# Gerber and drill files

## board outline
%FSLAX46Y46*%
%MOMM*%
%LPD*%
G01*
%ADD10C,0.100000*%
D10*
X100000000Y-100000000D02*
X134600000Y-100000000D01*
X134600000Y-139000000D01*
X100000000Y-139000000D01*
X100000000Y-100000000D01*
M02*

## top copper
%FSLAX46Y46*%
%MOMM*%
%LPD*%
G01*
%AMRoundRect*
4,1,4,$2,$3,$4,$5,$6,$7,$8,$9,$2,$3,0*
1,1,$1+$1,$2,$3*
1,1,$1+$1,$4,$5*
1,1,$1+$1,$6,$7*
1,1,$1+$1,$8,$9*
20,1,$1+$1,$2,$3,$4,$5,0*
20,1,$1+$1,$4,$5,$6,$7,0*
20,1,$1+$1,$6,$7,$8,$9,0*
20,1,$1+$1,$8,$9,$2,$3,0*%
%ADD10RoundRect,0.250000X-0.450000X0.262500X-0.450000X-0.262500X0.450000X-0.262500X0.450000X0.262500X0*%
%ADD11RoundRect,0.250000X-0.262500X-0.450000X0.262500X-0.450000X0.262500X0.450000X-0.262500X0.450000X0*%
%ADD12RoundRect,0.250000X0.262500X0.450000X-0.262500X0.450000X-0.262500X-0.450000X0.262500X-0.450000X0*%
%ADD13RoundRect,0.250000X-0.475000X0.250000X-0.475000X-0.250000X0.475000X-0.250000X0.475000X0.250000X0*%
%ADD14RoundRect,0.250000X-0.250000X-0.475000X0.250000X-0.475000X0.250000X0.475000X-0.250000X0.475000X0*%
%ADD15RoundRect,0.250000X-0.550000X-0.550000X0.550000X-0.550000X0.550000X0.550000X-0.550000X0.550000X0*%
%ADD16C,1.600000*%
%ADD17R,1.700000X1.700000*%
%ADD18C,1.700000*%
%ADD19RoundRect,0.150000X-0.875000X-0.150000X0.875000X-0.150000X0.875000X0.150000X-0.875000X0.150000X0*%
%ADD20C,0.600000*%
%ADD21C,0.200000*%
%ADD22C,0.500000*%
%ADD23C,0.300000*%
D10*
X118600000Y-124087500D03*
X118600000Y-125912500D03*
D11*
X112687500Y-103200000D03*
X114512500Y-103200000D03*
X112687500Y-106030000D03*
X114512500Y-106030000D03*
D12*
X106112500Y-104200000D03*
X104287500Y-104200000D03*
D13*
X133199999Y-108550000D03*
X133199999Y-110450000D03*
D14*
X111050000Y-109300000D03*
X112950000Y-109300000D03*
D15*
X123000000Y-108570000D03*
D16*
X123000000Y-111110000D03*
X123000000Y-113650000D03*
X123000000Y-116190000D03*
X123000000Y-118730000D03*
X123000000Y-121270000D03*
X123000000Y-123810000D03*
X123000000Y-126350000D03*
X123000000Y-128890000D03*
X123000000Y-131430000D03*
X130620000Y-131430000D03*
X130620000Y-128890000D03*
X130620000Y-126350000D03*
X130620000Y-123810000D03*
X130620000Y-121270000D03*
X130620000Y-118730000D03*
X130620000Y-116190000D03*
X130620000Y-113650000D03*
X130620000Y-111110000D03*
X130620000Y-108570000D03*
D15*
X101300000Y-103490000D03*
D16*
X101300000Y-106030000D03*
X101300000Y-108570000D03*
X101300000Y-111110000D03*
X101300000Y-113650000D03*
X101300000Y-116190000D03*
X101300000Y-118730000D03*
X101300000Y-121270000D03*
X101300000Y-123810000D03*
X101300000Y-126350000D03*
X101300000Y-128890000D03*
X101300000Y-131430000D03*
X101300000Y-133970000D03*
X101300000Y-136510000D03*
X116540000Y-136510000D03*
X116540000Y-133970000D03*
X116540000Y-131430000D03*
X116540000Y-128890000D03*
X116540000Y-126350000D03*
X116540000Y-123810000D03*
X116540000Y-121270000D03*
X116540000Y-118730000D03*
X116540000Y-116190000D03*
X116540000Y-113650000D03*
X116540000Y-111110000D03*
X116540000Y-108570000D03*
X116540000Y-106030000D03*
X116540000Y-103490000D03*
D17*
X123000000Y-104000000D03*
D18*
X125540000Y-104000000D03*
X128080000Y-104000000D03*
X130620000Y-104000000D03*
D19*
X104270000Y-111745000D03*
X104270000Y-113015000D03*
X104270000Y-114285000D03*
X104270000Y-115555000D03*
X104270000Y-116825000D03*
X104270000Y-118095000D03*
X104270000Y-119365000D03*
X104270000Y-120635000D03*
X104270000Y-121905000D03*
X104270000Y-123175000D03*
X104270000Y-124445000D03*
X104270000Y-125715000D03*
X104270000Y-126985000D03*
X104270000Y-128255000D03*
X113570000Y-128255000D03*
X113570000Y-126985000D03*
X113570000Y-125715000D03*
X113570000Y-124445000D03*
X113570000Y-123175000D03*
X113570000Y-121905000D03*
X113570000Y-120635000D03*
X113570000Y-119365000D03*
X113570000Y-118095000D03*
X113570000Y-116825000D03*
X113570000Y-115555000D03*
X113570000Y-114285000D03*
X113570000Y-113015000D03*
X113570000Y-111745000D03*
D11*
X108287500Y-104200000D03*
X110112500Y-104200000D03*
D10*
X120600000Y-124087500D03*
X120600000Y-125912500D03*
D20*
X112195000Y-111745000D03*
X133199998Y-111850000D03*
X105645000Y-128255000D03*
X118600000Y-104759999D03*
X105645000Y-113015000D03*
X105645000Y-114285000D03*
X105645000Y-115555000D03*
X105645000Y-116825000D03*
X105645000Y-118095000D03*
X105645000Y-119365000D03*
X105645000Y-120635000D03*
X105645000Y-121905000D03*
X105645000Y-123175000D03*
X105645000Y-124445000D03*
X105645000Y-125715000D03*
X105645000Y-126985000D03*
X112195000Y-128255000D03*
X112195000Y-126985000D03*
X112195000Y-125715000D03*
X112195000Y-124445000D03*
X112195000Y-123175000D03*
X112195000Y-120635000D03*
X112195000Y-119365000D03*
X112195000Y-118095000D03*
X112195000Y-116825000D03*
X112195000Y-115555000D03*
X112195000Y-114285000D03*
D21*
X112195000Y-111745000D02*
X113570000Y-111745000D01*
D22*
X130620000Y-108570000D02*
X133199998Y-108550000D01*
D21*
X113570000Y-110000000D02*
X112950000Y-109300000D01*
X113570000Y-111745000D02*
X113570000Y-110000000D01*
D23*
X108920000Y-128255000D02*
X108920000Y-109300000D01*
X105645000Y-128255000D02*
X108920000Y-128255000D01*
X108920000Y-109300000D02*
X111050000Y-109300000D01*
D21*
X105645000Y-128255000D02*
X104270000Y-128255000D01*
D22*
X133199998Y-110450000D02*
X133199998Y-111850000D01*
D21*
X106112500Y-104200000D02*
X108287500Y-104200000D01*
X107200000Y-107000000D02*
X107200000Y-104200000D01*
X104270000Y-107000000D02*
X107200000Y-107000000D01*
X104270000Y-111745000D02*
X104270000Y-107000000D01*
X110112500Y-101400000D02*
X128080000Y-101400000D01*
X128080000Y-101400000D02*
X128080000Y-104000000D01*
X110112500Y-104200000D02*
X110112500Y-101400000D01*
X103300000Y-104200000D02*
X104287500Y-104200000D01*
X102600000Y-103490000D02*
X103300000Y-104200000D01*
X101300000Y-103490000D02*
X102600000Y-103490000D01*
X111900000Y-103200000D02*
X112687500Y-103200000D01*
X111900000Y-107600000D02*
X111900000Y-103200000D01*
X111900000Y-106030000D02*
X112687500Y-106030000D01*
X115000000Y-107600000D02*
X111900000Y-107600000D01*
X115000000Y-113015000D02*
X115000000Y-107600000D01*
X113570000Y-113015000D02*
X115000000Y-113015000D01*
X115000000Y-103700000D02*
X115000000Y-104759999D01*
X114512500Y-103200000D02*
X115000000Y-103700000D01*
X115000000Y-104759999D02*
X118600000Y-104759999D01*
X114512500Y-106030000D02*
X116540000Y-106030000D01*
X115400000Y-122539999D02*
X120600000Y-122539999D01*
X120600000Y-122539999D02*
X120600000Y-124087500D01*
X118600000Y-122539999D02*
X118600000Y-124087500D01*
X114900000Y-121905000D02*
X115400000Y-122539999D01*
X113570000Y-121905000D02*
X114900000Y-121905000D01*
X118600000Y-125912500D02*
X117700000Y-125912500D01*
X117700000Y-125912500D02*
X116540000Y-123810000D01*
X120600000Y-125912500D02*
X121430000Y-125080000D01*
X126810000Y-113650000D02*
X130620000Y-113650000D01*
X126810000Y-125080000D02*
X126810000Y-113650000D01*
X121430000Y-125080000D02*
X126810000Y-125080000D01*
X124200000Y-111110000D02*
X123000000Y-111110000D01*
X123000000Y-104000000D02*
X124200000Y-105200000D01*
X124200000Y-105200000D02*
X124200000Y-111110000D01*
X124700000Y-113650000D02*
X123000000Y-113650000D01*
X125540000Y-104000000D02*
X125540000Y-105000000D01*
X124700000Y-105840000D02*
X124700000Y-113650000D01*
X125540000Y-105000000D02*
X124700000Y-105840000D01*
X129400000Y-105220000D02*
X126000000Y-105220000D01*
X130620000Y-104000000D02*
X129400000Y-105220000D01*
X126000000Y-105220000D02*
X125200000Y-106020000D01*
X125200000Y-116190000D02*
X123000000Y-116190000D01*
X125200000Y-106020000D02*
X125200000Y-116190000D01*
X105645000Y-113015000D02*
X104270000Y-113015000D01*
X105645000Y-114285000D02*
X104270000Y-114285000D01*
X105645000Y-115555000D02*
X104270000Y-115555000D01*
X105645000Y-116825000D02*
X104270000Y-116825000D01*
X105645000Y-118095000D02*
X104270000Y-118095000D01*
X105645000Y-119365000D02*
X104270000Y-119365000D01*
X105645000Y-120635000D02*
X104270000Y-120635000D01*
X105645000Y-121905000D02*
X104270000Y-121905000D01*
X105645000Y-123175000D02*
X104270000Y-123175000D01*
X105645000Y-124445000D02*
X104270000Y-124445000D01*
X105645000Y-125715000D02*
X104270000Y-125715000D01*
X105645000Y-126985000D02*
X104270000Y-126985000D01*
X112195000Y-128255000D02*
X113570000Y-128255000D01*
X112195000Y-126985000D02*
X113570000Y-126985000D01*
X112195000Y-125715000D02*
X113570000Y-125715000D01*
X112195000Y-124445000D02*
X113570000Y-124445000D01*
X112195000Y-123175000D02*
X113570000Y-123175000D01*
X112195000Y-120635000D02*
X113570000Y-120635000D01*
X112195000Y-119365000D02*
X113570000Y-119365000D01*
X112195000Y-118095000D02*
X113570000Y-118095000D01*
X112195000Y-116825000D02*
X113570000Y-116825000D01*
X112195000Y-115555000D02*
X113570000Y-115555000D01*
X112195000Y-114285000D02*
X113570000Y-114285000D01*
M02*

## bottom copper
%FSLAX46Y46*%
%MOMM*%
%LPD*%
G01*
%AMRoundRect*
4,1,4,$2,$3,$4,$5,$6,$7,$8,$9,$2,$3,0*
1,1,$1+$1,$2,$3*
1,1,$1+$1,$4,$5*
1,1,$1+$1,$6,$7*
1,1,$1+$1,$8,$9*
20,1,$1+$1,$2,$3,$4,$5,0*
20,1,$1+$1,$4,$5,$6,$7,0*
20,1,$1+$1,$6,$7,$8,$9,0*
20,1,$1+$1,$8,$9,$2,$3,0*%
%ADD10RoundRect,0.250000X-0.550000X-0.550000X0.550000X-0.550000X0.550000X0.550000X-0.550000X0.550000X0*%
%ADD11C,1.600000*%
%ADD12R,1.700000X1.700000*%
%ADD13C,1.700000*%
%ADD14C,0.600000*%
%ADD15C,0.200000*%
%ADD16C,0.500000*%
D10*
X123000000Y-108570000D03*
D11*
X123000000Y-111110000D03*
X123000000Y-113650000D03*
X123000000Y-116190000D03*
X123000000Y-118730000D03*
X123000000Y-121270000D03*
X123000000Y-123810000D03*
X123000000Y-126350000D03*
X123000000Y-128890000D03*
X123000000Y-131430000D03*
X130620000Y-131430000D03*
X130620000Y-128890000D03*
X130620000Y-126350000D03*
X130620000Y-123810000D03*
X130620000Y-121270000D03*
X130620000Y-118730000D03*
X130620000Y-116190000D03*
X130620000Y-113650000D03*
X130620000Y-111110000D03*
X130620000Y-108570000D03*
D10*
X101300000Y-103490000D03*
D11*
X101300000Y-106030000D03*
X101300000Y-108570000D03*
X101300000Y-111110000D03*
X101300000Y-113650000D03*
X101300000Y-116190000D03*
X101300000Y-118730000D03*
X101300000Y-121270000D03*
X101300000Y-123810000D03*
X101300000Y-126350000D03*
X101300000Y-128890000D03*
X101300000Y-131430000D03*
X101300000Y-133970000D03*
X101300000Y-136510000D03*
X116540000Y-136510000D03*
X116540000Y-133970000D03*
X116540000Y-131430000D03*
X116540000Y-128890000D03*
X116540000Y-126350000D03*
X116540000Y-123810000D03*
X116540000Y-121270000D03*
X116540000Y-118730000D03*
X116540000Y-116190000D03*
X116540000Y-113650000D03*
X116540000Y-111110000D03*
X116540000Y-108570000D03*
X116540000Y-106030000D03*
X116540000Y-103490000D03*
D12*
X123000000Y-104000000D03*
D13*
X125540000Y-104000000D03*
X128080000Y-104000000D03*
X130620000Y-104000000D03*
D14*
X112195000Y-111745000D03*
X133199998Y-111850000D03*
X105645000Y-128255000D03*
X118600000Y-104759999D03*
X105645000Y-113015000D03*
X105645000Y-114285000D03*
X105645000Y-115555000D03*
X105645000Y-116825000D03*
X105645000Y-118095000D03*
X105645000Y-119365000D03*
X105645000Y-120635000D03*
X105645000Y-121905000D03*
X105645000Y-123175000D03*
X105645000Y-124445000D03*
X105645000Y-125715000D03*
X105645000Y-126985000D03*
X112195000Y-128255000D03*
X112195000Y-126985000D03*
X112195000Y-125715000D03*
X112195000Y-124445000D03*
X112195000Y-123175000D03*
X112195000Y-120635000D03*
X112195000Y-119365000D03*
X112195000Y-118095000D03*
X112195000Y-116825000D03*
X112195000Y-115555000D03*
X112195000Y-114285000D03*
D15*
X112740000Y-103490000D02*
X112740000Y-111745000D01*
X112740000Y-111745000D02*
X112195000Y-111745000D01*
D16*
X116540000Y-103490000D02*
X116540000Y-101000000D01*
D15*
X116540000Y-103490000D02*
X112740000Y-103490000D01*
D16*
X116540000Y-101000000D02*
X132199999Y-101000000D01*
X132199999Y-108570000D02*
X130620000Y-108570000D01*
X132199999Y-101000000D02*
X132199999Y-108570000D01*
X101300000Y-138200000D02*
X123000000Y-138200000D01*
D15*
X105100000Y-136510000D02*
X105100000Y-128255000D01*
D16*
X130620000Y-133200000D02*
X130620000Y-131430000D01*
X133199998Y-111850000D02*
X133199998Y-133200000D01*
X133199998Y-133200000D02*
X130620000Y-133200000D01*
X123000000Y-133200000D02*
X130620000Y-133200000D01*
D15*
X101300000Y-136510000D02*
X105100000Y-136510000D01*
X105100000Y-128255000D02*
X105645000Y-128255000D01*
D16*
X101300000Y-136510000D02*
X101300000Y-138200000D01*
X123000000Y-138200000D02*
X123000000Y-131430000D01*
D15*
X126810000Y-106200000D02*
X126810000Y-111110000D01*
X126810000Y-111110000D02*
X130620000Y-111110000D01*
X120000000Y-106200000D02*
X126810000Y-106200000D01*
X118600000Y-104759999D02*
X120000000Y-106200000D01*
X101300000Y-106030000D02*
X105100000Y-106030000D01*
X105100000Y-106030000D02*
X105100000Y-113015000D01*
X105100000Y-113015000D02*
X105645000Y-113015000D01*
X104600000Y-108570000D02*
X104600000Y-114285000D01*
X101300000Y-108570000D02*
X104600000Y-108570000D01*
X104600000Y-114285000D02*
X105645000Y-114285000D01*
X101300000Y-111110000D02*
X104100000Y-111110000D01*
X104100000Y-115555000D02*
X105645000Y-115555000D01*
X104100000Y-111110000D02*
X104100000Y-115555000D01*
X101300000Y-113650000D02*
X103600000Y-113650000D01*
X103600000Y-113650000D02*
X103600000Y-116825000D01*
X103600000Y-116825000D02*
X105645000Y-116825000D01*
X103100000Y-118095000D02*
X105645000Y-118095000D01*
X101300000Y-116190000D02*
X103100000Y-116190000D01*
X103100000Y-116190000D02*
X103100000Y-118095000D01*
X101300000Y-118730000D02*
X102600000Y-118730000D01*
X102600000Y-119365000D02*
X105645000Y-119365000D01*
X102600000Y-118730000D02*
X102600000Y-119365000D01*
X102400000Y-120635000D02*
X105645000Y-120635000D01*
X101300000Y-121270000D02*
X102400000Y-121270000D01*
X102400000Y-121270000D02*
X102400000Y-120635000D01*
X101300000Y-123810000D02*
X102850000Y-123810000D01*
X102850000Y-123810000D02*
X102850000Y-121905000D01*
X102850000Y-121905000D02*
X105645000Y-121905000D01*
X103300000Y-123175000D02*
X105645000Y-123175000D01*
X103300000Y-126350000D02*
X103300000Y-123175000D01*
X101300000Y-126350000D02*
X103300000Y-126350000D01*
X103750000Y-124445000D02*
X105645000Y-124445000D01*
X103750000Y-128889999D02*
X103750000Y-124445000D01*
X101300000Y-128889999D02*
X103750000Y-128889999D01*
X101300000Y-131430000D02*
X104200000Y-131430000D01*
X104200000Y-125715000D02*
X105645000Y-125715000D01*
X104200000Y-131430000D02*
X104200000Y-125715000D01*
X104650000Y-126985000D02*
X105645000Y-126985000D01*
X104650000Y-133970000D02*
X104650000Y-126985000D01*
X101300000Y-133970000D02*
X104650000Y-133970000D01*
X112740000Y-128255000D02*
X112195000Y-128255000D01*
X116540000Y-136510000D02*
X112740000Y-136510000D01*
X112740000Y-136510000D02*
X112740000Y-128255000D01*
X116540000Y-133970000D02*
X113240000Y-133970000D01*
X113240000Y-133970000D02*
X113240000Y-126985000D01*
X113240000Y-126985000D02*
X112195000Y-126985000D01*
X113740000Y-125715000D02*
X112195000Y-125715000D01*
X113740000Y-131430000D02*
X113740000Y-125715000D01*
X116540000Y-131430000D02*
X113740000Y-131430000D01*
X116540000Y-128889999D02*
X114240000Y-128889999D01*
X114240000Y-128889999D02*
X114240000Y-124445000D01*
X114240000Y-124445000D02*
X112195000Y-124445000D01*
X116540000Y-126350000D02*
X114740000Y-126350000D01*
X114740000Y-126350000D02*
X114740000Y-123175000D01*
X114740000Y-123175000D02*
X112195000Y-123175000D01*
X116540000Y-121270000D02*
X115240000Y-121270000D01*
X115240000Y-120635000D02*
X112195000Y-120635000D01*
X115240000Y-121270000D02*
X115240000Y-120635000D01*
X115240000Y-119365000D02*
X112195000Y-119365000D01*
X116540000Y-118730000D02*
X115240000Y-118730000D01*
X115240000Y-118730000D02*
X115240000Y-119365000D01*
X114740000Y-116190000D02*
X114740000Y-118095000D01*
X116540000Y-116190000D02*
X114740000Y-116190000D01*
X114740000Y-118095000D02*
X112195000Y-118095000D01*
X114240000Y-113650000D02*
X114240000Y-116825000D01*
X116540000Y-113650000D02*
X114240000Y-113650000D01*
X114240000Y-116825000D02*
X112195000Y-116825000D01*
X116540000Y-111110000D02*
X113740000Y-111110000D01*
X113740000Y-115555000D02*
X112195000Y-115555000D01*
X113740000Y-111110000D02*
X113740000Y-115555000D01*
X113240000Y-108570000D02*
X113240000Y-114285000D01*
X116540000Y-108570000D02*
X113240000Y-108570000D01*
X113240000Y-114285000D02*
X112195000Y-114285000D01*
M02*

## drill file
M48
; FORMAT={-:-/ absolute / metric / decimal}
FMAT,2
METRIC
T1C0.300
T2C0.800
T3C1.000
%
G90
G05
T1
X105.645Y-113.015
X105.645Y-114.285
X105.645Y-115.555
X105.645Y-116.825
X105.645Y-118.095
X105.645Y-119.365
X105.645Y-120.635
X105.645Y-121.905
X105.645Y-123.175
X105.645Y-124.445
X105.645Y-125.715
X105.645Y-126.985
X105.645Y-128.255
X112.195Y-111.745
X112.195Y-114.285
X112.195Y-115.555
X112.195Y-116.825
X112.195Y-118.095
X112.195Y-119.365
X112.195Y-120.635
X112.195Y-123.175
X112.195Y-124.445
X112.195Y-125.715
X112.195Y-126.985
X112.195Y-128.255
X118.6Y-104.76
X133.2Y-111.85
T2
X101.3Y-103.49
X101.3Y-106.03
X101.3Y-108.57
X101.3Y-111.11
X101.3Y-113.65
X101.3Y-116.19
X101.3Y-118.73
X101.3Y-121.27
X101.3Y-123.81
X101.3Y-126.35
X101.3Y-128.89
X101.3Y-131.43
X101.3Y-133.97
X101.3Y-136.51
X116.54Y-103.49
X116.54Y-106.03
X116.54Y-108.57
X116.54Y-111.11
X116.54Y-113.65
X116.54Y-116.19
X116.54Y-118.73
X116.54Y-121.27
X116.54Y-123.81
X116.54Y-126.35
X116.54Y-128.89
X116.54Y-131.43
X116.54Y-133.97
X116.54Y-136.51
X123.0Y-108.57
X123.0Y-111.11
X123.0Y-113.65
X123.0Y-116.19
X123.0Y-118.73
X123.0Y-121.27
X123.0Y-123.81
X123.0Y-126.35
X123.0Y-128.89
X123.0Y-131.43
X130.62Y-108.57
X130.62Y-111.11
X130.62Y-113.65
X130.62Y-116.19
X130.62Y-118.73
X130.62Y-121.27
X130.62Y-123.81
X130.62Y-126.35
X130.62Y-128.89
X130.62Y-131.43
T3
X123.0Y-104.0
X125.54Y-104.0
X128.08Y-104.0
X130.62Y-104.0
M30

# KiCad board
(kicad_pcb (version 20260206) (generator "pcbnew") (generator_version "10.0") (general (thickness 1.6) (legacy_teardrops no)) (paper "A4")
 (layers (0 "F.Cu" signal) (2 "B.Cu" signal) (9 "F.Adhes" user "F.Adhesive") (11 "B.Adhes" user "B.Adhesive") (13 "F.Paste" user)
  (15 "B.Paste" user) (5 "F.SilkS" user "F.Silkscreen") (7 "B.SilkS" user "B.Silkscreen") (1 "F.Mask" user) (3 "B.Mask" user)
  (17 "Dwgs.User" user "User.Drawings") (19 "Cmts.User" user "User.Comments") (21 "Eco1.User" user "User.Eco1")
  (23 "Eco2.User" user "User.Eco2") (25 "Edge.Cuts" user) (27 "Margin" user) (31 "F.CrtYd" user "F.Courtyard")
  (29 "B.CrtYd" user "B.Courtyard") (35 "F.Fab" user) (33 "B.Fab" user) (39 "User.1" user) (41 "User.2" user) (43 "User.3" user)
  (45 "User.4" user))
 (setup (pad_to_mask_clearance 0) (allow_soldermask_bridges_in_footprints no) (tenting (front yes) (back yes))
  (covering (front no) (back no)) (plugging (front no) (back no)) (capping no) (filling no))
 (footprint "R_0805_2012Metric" (layer "F.Cu") (at 118.6 125 -90)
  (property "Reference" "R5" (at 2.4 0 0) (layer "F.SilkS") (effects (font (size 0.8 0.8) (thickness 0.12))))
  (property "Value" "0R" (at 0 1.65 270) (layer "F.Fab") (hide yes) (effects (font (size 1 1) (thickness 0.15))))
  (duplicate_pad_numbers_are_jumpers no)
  (pad "1" smd roundrect (at -0.9125 0 270) (size 1.025 1.4) (layers "F.Cu" "F.Mask" "F.Paste") (roundrect_rratio 0.243902) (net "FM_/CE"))
  (pad "2" smd roundrect (at 0.9125 0 270) (size 1.025 1.4) (layers "F.Cu" "F.Mask" "F.Paste") (roundrect_rratio 0.243902) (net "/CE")))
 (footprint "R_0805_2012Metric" (layer "F.Cu") (at 113.6 103.2)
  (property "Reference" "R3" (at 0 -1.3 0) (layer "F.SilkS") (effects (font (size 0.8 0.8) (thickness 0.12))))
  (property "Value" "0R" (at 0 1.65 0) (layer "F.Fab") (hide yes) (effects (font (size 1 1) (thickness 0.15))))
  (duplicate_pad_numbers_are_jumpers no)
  (pad "1" smd roundrect (at -0.9125 0) (size 1.025 1.4) (layers "F.Cu" "F.Mask" "F.Paste") (roundrect_rratio 0.243902) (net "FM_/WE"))
  (pad "2" smd roundrect (at 0.9125 0) (size 1.025 1.4) (layers "F.Cu" "F.Mask" "F.Paste") (roundrect_rratio 0.243902) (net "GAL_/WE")))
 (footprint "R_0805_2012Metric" (layer "F.Cu") (at 113.6 106.03)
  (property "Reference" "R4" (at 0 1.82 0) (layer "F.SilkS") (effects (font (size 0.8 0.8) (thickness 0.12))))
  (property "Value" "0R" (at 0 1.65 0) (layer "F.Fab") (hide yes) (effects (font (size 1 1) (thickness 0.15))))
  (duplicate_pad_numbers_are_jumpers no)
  (pad "1" smd roundrect (at -0.9125 0) (size 1.025 1.4) (layers "F.Cu" "F.Mask" "F.Paste") (roundrect_rratio 0.243902) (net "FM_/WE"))
  (pad "2" smd roundrect (at 0.9125 0) (size 1.025 1.4) (layers "F.Cu" "F.Mask" "F.Paste") (roundrect_rratio 0.243902) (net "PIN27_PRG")))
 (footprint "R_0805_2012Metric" (layer "F.Cu") (at 105.2 104.2 180)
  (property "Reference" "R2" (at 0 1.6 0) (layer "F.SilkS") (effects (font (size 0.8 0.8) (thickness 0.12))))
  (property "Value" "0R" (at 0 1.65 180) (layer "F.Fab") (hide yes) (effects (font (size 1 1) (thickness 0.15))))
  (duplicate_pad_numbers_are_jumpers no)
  (pad "1" smd roundrect (at -0.9125 0 180) (size 1.025 1.4) (layers "F.Cu" "F.Mask" "F.Paste") (roundrect_rratio 0.243902) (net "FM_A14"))
  (pad "2" smd roundrect (at 0.9125 0 180) (size 1.025 1.4) (layers "F.Cu" "F.Mask" "F.Paste") (roundrect_rratio 0.243902) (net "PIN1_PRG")))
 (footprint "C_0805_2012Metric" (layer "F.Cu") (at 133.199999 109.5 -90)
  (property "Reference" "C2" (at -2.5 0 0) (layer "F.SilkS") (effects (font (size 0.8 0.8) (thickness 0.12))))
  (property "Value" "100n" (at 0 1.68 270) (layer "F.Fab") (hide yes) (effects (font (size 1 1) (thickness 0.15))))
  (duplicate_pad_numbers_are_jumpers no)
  (pad "1" smd roundrect (at -0.95 0 270) (size 1 1.45) (layers "F.Cu" "F.Mask" "F.Paste") (roundrect_rratio 0.25) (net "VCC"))
  (pad "2" smd roundrect (at 0.95 0 270) (size 1 1.45) (layers "F.Cu" "F.Mask" "F.Paste") (roundrect_rratio 0.25) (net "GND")))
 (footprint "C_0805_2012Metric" (layer "F.Cu") (at 112 109.3)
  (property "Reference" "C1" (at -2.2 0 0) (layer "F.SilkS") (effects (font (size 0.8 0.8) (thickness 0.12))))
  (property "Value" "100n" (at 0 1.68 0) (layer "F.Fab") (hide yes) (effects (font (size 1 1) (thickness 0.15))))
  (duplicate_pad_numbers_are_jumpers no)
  (pad "1" smd roundrect (at -0.95 0) (size 1 1.45) (layers "F.Cu" "F.Mask" "F.Paste") (roundrect_rratio 0.25) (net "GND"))
  (pad "2" smd roundrect (at 0.95 0) (size 1 1.45) (layers "F.Cu" "F.Mask" "F.Paste") (roundrect_rratio 0.25) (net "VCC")))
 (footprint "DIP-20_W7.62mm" (layer "F.Cu") (at 123 108.57)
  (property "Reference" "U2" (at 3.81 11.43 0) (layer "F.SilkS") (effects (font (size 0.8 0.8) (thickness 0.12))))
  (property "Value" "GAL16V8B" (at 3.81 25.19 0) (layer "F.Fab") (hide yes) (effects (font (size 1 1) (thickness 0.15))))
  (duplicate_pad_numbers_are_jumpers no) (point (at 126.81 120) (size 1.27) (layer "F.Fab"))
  (pad "1" thru_hole roundrect (at 0 0) (size 1.6 1.6) (drill 0.8) (layers "*.Cu" "*.Mask") (remove_unused_layers no)
   (roundrect_rratio 0.15625))
  (pad "2" thru_hole circle (at 0 2.54) (size 1.6 1.6) (drill 0.8) (layers "*.Cu" "*.Mask") (remove_unused_layers no) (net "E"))
  (pad "3" thru_hole circle (at 0 5.08) (size 1.6 1.6) (drill 0.8) (layers "*.Cu" "*.Mask") (remove_unused_layers no) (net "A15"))
  (pad "4" thru_hole circle (at 0 7.62) (size 1.6 1.6) (drill 0.8) (layers "*.Cu" "*.Mask") (remove_unused_layers no) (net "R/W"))
  (pad "5" thru_hole circle (at 0 10.16) (size 1.6 1.6) (drill 0.8) (layers "*.Cu" "*.Mask") (remove_unused_layers no))
  (pad "6" thru_hole circle (at 0 12.7) (size 1.6 1.6) (drill 0.8) (layers "*.Cu" "*.Mask") (remove_unused_layers no))
  (pad "7" thru_hole circle (at 0 15.24) (size 1.6 1.6) (drill 0.8) (layers "*.Cu" "*.Mask") (remove_unused_layers no))
  (pad "8" thru_hole circle (at 0 17.78) (size 1.6 1.6) (drill 0.8) (layers "*.Cu" "*.Mask") (remove_unused_layers no))
  (pad "9" thru_hole circle (at 0 20.32) (size 1.6 1.6) (drill 0.8) (layers "*.Cu" "*.Mask") (remove_unused_layers no))
  (pad "10" thru_hole circle (at 0 22.86) (size 1.6 1.6) (drill 0.8) (layers "*.Cu" "*.Mask") (remove_unused_layers no) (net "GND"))
  (pad "11" thru_hole circle (at 7.62 22.86) (size 1.6 1.6) (drill 0.8) (layers "*.Cu" "*.Mask") (remove_unused_layers no) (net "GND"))
  (pad "12" thru_hole circle (at 7.62 20.32) (size 1.6 1.6) (drill 0.8) (layers "*.Cu" "*.Mask") (remove_unused_layers no))
  (pad "13" thru_hole circle (at 7.62 17.78) (size 1.6 1.6) (drill 0.8) (layers "*.Cu" "*.Mask") (remove_unused_layers no))
  (pad "14" thru_hole circle (at 7.62 15.24) (size 1.6 1.6) (drill 0.8) (layers "*.Cu" "*.Mask") (remove_unused_layers no))
  (pad "15" thru_hole circle (at 7.62 12.7) (size 1.6 1.6) (drill 0.8) (layers "*.Cu" "*.Mask") (remove_unused_layers no))
  (pad "16" thru_hole circle (at 7.62 10.16) (size 1.6 1.6) (drill 0.8) (layers "*.Cu" "*.Mask") (remove_unused_layers no))
  (pad "17" thru_hole circle (at 7.62 7.62) (size 1.6 1.6) (drill 0.8) (layers "*.Cu" "*.Mask") (remove_unused_layers no))
  (pad "18" thru_hole circle (at 7.62 5.08) (size 1.6 1.6) (drill 0.8) (layers "*.Cu" "*.Mask") (remove_unused_layers no) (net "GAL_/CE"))
  (pad "19" thru_hole circle (at 7.62 2.54) (size 1.6 1.6) (drill 0.8) (layers "*.Cu" "*.Mask") (remove_unused_layers no) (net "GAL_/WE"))
  (pad "20" thru_hole circle (at 7.62 0) (size 1.6 1.6) (drill 0.8) (layers "*.Cu" "*.Mask") (remove_unused_layers no) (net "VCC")))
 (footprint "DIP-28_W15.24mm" (layer "F.Cu") (at 101.3 103.49)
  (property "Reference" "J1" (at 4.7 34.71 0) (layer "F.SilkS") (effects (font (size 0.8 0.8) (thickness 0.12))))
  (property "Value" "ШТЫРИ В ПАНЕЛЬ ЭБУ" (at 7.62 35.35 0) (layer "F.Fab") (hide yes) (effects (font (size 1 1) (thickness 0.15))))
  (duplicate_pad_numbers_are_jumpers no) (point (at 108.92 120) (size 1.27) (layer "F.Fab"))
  (pad "1" thru_hole roundrect (at 0 0) (size 1.6 1.6) (drill 0.8) (layers "*.Cu" "*.Mask") (remove_unused_layers no)
   (roundrect_rratio 0.15625) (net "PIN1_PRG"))
  (pad "2" thru_hole circle (at 0 2.54) (size 1.6 1.6) (drill 0.8) (layers "*.Cu" "*.Mask") (remove_unused_layers no) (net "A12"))
  (pad "3" thru_hole circle (at 0 5.08) (size 1.6 1.6) (drill 0.8) (layers "*.Cu" "*.Mask") (remove_unused_layers no) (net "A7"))
  (pad "4" thru_hole circle (at 0 7.62) (size 1.6 1.6) (drill 0.8) (layers "*.Cu" "*.Mask") (remove_unused_layers no) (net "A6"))
  (pad "5" thru_hole circle (at 0 10.16) (size 1.6 1.6) (drill 0.8) (layers "*.Cu" "*.Mask") (remove_unused_layers no) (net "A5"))
  (pad "6" thru_hole circle (at 0 12.7) (size 1.6 1.6) (drill 0.8) (layers "*.Cu" "*.Mask") (remove_unused_layers no) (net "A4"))
  (pad "7" thru_hole circle (at 0 15.24) (size 1.6 1.6) (drill 0.8) (layers "*.Cu" "*.Mask") (remove_unused_layers no) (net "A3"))
  (pad "8" thru_hole circle (at 0 17.78) (size 1.6 1.6) (drill 0.8) (layers "*.Cu" "*.Mask") (remove_unused_layers no) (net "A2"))
  (pad "9" thru_hole circle (at 0 20.32) (size 1.6 1.6) (drill 0.8) (layers "*.Cu" "*.Mask") (remove_unused_layers no) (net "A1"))
  (pad "10" thru_hole circle (at 0 22.86) (size 1.6 1.6) (drill 0.8) (layers "*.Cu" "*.Mask") (remove_unused_layers no) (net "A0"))
  (pad "11" thru_hole circle (at 0 25.4) (size 1.6 1.6) (drill 0.8) (layers "*.Cu" "*.Mask") (remove_unused_layers no) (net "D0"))
  (pad "12" thru_hole circle (at 0 27.94) (size 1.6 1.6) (drill 0.8) (layers "*.Cu" "*.Mask") (remove_unused_layers no) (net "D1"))
  (pad "13" thru_hole circle (at 0 30.48) (size 1.6 1.6) (drill 0.8) (layers "*.Cu" "*.Mask") (remove_unused_layers no) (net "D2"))
  (pad "14" thru_hole circle (at 0 33.02) (size 1.6 1.6) (drill 0.8) (layers "*.Cu" "*.Mask") (remove_unused_layers no) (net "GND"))
  (pad "15" thru_hole circle (at 15.24 33.02) (size 1.6 1.6) (drill 0.8) (layers "*.Cu" "*.Mask") (remove_unused_layers no) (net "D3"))
  (pad "16" thru_hole circle (at 15.24 30.48) (size 1.6 1.6) (drill 0.8) (layers "*.Cu" "*.Mask") (remove_unused_layers no) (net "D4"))
  (pad "17" thru_hole circle (at 15.24 27.94) (size 1.6 1.6) (drill 0.8) (layers "*.Cu" "*.Mask") (remove_unused_layers no) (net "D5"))
  (pad "18" thru_hole circle (at 15.24 25.4) (size 1.6 1.6) (drill 0.8) (layers "*.Cu" "*.Mask") (remove_unused_layers no) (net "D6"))
  (pad "19" thru_hole circle (at 15.24 22.86) (size 1.6 1.6) (drill 0.8) (layers "*.Cu" "*.Mask") (remove_unused_layers no) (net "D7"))
  (pad "20" thru_hole circle (at 15.24 20.32) (size 1.6 1.6) (drill 0.8) (layers "*.Cu" "*.Mask") (remove_unused_layers no) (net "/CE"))
  (pad "21" thru_hole circle (at 15.24 17.78) (size 1.6 1.6) (drill 0.8) (layers "*.Cu" "*.Mask") (remove_unused_layers no) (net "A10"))
  (pad "22" thru_hole circle (at 15.24 15.24) (size 1.6 1.6) (drill 0.8) (layers "*.Cu" "*.Mask") (remove_unused_layers no) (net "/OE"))
  (pad "23" thru_hole circle (at 15.24 12.7) (size 1.6 1.6) (drill 0.8) (layers "*.Cu" "*.Mask") (remove_unused_layers no) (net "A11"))
  (pad "24" thru_hole circle (at 15.24 10.16) (size 1.6 1.6) (drill 0.8) (layers "*.Cu" "*.Mask") (remove_unused_layers no) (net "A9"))
  (pad "25" thru_hole circle (at 15.24 7.62) (size 1.6 1.6) (drill 0.8) (layers "*.Cu" "*.Mask") (remove_unused_layers no) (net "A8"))
  (pad "26" thru_hole circle (at 15.24 5.08) (size 1.6 1.6) (drill 0.8) (layers "*.Cu" "*.Mask") (remove_unused_layers no) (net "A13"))
  (pad "27" thru_hole circle (at 15.24 2.54) (size 1.6 1.6) (drill 0.8) (layers "*.Cu" "*.Mask") (remove_unused_layers no) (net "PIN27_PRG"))
  (pad "28" thru_hole circle (at 15.24 0) (size 1.6 1.6) (drill 0.8) (layers "*.Cu" "*.Mask") (remove_unused_layers no) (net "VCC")))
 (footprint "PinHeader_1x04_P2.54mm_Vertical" (layer "F.Cu") (at 123 104 90)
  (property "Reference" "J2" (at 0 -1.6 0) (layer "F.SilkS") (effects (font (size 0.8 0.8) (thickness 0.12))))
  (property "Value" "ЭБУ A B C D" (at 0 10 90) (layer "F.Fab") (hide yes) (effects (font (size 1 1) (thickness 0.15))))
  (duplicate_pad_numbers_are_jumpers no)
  (pad "1" thru_hole rect (at 0 0 90) (size 1.7 1.7) (drill 1) (layers "*.Cu" "*.Mask") (remove_unused_layers no) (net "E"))
  (pad "2" thru_hole circle (at 0 2.54 90) (size 1.7 1.7) (drill 1) (layers "*.Cu" "*.Mask") (remove_unused_layers no) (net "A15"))
  (pad "3" thru_hole circle (at 0 5.08 90) (size 1.7 1.7) (drill 1) (layers "*.Cu" "*.Mask") (remove_unused_layers no) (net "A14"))
  (pad "4" thru_hole circle (at 0 7.62 90) (size 1.7 1.7) (drill 1) (layers "*.Cu" "*.Mask") (remove_unused_layers no) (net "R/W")))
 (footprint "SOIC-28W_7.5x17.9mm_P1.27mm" (layer "F.Cu") (at 108.92 120)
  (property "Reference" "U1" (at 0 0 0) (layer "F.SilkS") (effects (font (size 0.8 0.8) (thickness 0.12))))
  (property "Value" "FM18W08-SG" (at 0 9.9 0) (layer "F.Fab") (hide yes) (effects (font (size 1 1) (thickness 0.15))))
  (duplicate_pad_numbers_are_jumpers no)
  (pad "1" smd roundrect (at -4.65 -8.255) (size 2.05 0.6) (layers "F.Cu" "F.Mask" "F.Paste") (roundrect_rratio 0.25) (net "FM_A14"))
  (pad "2" smd roundrect (at -4.65 -6.985) (size 2.05 0.6) (layers "F.Cu" "F.Mask" "F.Paste") (roundrect_rratio 0.25) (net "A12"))
  (pad "3" smd roundrect (at -4.65 -5.715) (size 2.05 0.6) (layers "F.Cu" "F.Mask" "F.Paste") (roundrect_rratio 0.25) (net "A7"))
  (pad "4" smd roundrect (at -4.65 -4.445) (size 2.05 0.6) (layers "F.Cu" "F.Mask" "F.Paste") (roundrect_rratio 0.25) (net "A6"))
  (pad "5" smd roundrect (at -4.65 -3.175) (size 2.05 0.6) (layers "F.Cu" "F.Mask" "F.Paste") (roundrect_rratio 0.25) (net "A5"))
  (pad "6" smd roundrect (at -4.65 -1.905) (size 2.05 0.6) (layers "F.Cu" "F.Mask" "F.Paste") (roundrect_rratio 0.25) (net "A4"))
  (pad "7" smd roundrect (at -4.65 -0.635) (size 2.05 0.6) (layers "F.Cu" "F.Mask" "F.Paste") (roundrect_rratio 0.25) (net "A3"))
  (pad "8" smd roundrect (at -4.65 0.635) (size 2.05 0.6) (layers "F.Cu" "F.Mask" "F.Paste") (roundrect_rratio 0.25) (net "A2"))
  (pad "9" smd roundrect (at -4.65 1.905) (size 2.05 0.6) (layers "F.Cu" "F.Mask" "F.Paste") (roundrect_rratio 0.25) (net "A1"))
  (pad "10" smd roundrect (at -4.65 3.175) (size 2.05 0.6) (layers "F.Cu" "F.Mask" "F.Paste") (roundrect_rratio 0.25) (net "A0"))
  (pad "11" smd roundrect (at -4.65 4.445) (size 2.05 0.6) (layers "F.Cu" "F.Mask" "F.Paste") (roundrect_rratio 0.25) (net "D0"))
  (pad "12" smd roundrect (at -4.65 5.715) (size 2.05 0.6) (layers "F.Cu" "F.Mask" "F.Paste") (roundrect_rratio 0.25) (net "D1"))
  (pad "13" smd roundrect (at -4.65 6.985) (size 2.05 0.6) (layers "F.Cu" "F.Mask" "F.Paste") (roundrect_rratio 0.25) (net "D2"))
  (pad "14" smd roundrect (at -4.65 8.255) (size 2.05 0.6) (layers "F.Cu" "F.Mask" "F.Paste") (roundrect_rratio 0.25) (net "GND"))
  (pad "15" smd roundrect (at 4.65 8.255) (size 2.05 0.6) (layers "F.Cu" "F.Mask" "F.Paste") (roundrect_rratio 0.25) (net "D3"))
  (pad "16" smd roundrect (at 4.65 6.985) (size 2.05 0.6) (layers "F.Cu" "F.Mask" "F.Paste") (roundrect_rratio 0.25) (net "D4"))
  (pad "17" smd roundrect (at 4.65 5.715) (size 2.05 0.6) (layers "F.Cu" "F.Mask" "F.Paste") (roundrect_rratio 0.25) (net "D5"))
  (pad "18" smd roundrect (at 4.65 4.445) (size 2.05 0.6) (layers "F.Cu" "F.Mask" "F.Paste") (roundrect_rratio 0.25) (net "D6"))
  (pad "19" smd roundrect (at 4.65 3.175) (size 2.05 0.6) (layers "F.Cu" "F.Mask" "F.Paste") (roundrect_rratio 0.25) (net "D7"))
  (pad "20" smd roundrect (at 4.65 1.905) (size 2.05 0.6) (layers "F.Cu" "F.Mask" "F.Paste") (roundrect_rratio 0.25) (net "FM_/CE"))
  (pad "21" smd roundrect (at 4.65 0.635) (size 2.05 0.6) (layers "F.Cu" "F.Mask" "F.Paste") (roundrect_rratio 0.25) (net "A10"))
  (pad "22" smd roundrect (at 4.65 -0.635) (size 2.05 0.6) (layers "F.Cu" "F.Mask" "F.Paste") (roundrect_rratio 0.25) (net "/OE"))
  (pad "23" smd roundrect (at 4.65 -1.905) (size 2.05 0.6) (layers "F.Cu" "F.Mask" "F.Paste") (roundrect_rratio 0.25) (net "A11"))
  (pad "24" smd roundrect (at 4.65 -3.175) (size 2.05 0.6) (layers "F.Cu" "F.Mask" "F.Paste") (roundrect_rratio 0.25) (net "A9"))
  (pad "25" smd roundrect (at 4.65 -4.445) (size 2.05 0.6) (layers "F.Cu" "F.Mask" "F.Paste") (roundrect_rratio 0.25) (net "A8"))
  (pad "26" smd roundrect (at 4.65 -5.715) (size 2.05 0.6) (layers "F.Cu" "F.Mask" "F.Paste") (roundrect_rratio 0.25) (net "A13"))
  (pad "27" smd roundrect (at 4.65 -6.985) (size 2.05 0.6) (layers "F.Cu" "F.Mask" "F.Paste") (roundrect_rratio 0.25) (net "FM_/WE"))
  (pad "28" smd roundrect (at 4.65 -8.255) (size 2.05 0.6) (layers "F.Cu" "F.Mask" "F.Paste") (roundrect_rratio 0.25) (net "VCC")))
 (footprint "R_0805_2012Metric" (layer "F.Cu") (at 109.2 104.2)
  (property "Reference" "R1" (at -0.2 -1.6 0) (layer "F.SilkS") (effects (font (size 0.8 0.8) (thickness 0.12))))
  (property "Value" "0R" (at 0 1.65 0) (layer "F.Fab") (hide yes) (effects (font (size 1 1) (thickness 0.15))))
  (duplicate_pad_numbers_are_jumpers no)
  (pad "1" smd roundrect (at -0.9125 0) (size 1.025 1.4) (layers "F.Cu" "F.Mask" "F.Paste") (roundrect_rratio 0.243902) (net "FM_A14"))
  (pad "2" smd roundrect (at 0.9125 0) (size 1.025 1.4) (layers "F.Cu" "F.Mask" "F.Paste") (roundrect_rratio 0.243902) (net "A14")))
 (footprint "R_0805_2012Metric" (layer "F.Cu") (at 120.6 125 -90)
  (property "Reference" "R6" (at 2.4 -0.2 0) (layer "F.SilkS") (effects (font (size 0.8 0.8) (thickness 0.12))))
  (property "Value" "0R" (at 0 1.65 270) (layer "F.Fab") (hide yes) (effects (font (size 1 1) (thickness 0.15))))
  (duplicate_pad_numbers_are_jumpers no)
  (pad "1" smd roundrect (at -0.9125 0 270) (size 1.025 1.4) (layers "F.Cu" "F.Mask" "F.Paste") (roundrect_rratio 0.243902) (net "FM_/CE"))
  (pad "2" smd roundrect (at 0.9125 0 270) (size 1.025 1.4) (layers "F.Cu" "F.Mask" "F.Paste") (roundrect_rratio 0.243902) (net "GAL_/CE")))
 (gr_rect (start 100 100) (end 134.6 139) (stroke (width 0.1) (type default)) (fill no) (layer "Edge.Cuts"))
 (segment (start 112.195 111.745) (end 113.57 111.745) (width 0.2) (layer "F.Cu") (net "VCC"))
 (segment (start 130.62 108.57) (end 133.199998 108.55) (width 0.5) (layer "F.Cu") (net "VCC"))
 (segment (start 113.57 110) (end 112.95 109.3) (width 0.2) (layer "F.Cu") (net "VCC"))
 (segment (start 113.57 111.745) (end 113.57 110) (width 0.2) (layer "F.Cu") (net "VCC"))
 (via (at 112.195 111.745) (size 0.6) (drill 0.3) (layers "F.Cu" "B.Cu") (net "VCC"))
 (segment (start 112.74 103.49) (end 112.74 111.745) (width 0.2) (layer "B.Cu") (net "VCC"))
 (segment (start 112.74 111.745) (end 112.195 111.745) (width 0.2) (layer "B.Cu") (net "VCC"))
 (segment (start 116.54 103.49) (end 116.54 101) (width 0.5) (layer "B.Cu") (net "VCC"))
 (segment (start 116.54 103.49) (end 112.74 103.49) (width 0.2) (layer "B.Cu") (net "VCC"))
 (segment (start 116.54 101) (end 132.199999 101) (width 0.5) (layer "B.Cu") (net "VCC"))
 (segment (start 132.199999 108.57) (end 130.62 108.57) (width 0.5) (layer "B.Cu") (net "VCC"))
 (segment (start 132.199999 101) (end 132.199999 108.57) (width 0.5) (layer "B.Cu") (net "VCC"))
 (segment (start 108.92 128.255) (end 108.92 109.3) (width 0.3) (layer "F.Cu") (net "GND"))
 (segment (start 105.645 128.255) (end 108.92 128.255) (width 0.3) (layer "F.Cu") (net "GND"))
 (segment (start 108.92 109.3) (end 111.05 109.3) (width 0.3) (layer "F.Cu") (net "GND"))
 (segment (start 105.645 128.255) (end 104.27 128.255) (width 0.2) (layer "F.Cu") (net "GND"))
 (segment (start 133.199998 110.45) (end 133.199998 111.85) (width 0.5) (layer "F.Cu") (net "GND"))
 (via (at 133.199998 111.85) (size 0.6) (drill 0.3) (layers "F.Cu" "B.Cu") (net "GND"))
 (via (at 105.645 128.255) (size 0.6) (drill 0.3) (layers "F.Cu" "B.Cu") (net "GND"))
 (segment (start 101.3 138.2) (end 123 138.2) (width 0.5) (layer "B.Cu") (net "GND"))
 (segment (start 105.1 136.51) (end 105.1 128.255) (width 0.2) (layer "B.Cu") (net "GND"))
 (segment (start 130.62 133.2) (end 130.62 131.43) (width 0.5) (layer "B.Cu") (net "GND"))
 (segment (start 133.199998 111.85) (end 133.199998 133.2) (width 0.5) (layer "B.Cu") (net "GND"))
 (segment (start 133.199998 133.2) (end 130.62 133.2) (width 0.5) (layer "B.Cu") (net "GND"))
 (segment (start 123 133.2) (end 130.62 133.2) (width 0.5) (layer "B.Cu") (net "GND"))
 (segment (start 101.3 136.51) (end 105.1 136.51) (width 0.2) (layer "B.Cu") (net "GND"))
 (segment (start 105.1 128.255) (end 105.645 128.255) (width 0.2) (layer "B.Cu") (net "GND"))
 (segment (start 101.3 136.51) (end 101.3 138.2) (width 0.5) (layer "B.Cu") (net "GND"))
 (segment (start 123 138.2) (end 123 131.43) (width 0.5) (layer "B.Cu") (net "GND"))
 (segment (start 106.1125 104.2) (end 108.2875 104.2) (width 0.2) (layer "F.Cu") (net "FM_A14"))
 (segment (start 107.2 107) (end 107.2 104.2) (width 0.2) (layer "F.Cu") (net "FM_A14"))
 (segment (start 104.27 107) (end 107.2 107) (width 0.2) (layer "F.Cu") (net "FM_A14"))
 (segment (start 104.27 111.745) (end 104.27 107) (width 0.2) (layer "F.Cu") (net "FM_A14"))
 (segment (start 110.1125 101.4) (end 128.08 101.4) (width 0.2) (layer "F.Cu") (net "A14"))
 (segment (start 128.08 101.4) (end 128.08 104) (width 0.2) (layer "F.Cu") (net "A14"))
 (segment (start 110.1125 104.2) (end 110.1125 101.4) (width 0.2) (layer "F.Cu") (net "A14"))
 (segment (start 103.3 104.2) (end 104.2875 104.2) (width 0.2) (layer "F.Cu") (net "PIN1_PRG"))
 (segment (start 102.6 103.49) (end 103.3 104.2) (width 0.2) (layer "F.Cu") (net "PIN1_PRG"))
 (segment (start 101.3 103.49) (end 102.6 103.49) (width 0.2) (layer "F.Cu") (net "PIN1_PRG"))
 (segment (start 111.9 103.2) (end 112.6875 103.2) (width 0.2) (layer "F.Cu") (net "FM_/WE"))
 (segment (start 111.9 107.6) (end 111.9 103.2) (width 0.2) (layer "F.Cu") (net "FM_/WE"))
 (segment (start 111.9 106.03) (end 112.6875 106.03) (width 0.2) (layer "F.Cu") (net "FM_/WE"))
 (segment (start 115 107.6) (end 111.9 107.6) (width 0.2) (layer "F.Cu") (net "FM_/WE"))
 (segment (start 115 113.015) (end 115 107.6) (width 0.2) (layer "F.Cu") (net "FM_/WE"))
 (segment (start 113.57 113.015) (end 115 113.015) (width 0.2) (layer "F.Cu") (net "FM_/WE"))
 (segment (start 115 103.7) (end 115 104.759999) (width 0.2) (layer "F.Cu") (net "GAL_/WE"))
 (segment (start 114.5125 103.2) (end 115 103.7) (width 0.2) (layer "F.Cu") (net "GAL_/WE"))
 (segment (start 115 104.759999) (end 118.6 104.759999) (width 0.2) (layer "F.Cu") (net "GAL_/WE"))
 (via (at 118.6 104.759999) (size 0.6) (drill 0.3) (layers "F.Cu" "B.Cu") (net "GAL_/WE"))
 (segment (start 126.81 106.2) (end 126.81 111.11) (width 0.2) (layer "B.Cu") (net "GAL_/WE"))
 (segment (start 126.81 111.11) (end 130.62 111.11) (width 0.2) (layer "B.Cu") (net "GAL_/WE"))
 (segment (start 120 106.2) (end 126.81 106.2) (width 0.2) (layer "B.Cu") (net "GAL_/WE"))
 (segment (start 118.6 104.759999) (end 120 106.2) (width 0.2) (layer "B.Cu") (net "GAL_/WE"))
 (segment (start 114.5125 106.03) (end 116.54 106.03) (width 0.2) (layer "F.Cu") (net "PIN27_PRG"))
 (segment (start 115.4 122.539999) (end 120.6 122.539999) (width 0.2) (layer "F.Cu") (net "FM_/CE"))
 (segment (start 120.6 122.539999) (end 120.6 124.0875) (width 0.2) (layer "F.Cu") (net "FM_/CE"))
 (segment (start 118.6 122.539999) (end 118.6 124.0875) (width 0.2) (layer "F.Cu") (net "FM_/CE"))
 (segment (start 114.9 121.905) (end 115.4 122.539999) (width 0.2) (layer "F.Cu") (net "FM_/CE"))
 (segment (start 113.57 121.905) (end 114.9 121.905) (width 0.2) (layer "F.Cu") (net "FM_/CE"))
 (segment (start 118.6 125.9125) (end 117.7 125.9125) (width 0.2) (layer "F.Cu") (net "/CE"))
 (segment (start 117.7 125.9125) (end 116.54 123.81) (width 0.2) (layer "F.Cu") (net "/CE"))
 (segment (start 120.6 125.9125) (end 121.43 125.08) (width 0.2) (layer "F.Cu") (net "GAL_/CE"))
 (segment (start 126.81 113.65) (end 130.62 113.65) (width 0.2) (layer "F.Cu") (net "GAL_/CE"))
 (segment (start 126.81 125.08) (end 126.81 113.65) (width 0.2) (layer "F.Cu") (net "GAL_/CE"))
 (segment (start 121.43 125.08) (end 126.81 125.08) (width 0.2) (layer "F.Cu") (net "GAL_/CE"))
 (segment (start 124.2 111.11) (end 123 111.11) (width 0.2) (layer "F.Cu") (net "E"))
 (segment (start 123 104) (end 124.2 105.2) (width 0.2) (layer "F.Cu") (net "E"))
 (segment (start 124.2 105.2) (end 124.2 111.11) (width 0.2) (layer "F.Cu") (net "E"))
 (segment (start 124.7 113.65) (end 123 113.65) (width 0.2) (layer "F.Cu") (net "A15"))
 (segment (start 125.54 104) (end 125.54 105) (width 0.2) (layer "F.Cu") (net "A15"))
 (segment (start 124.7 105.84) (end 124.7 113.65) (width 0.2) (layer "F.Cu") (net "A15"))
 (segment (start 125.54 105) (end 124.7 105.84) (width 0.2) (layer "F.Cu") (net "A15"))
 (segment (start 129.4 105.22) (end 126 105.22) (width 0.2) (layer "F.Cu") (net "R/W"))
 (segment (start 130.62 104) (end 129.4 105.22) (width 0.2) (layer "F.Cu") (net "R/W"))
 (segment (start 126 105.22) (end 125.2 106.02) (width 0.2) (layer "F.Cu") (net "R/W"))
 (segment (start 125.2 116.19) (end 123 116.19) (width 0.2) (layer "F.Cu") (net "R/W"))
 (segment (start 125.2 106.02) (end 125.2 116.19) (width 0.2) (layer "F.Cu") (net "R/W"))
 (segment (start 105.645 113.015) (end 104.27 113.015) (width 0.2) (layer "F.Cu") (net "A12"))
 (via (at 105.645 113.015) (size 0.6) (drill 0.3) (layers "F.Cu" "B.Cu") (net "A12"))
 (segment (start 101.3 106.03) (end 105.1 106.03) (width 0.2) (layer "B.Cu") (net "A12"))
 (segment (start 105.1 106.03) (end 105.1 113.015) (width 0.2) (layer "B.Cu") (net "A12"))
 (segment (start 105.1 113.015) (end 105.645 113.015) (width 0.2) (layer "B.Cu") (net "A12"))
 (segment (start 105.645 114.285) (end 104.27 114.285) (width 0.2) (layer "F.Cu") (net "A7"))
 (via (at 105.645 114.285) (size 0.6) (drill 0.3) (layers "F.Cu" "B.Cu") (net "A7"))
 (segment (start 104.6 108.57) (end 104.6 114.285) (width 0.2) (layer "B.Cu") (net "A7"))
 (segment (start 101.3 108.57) (end 104.6 108.57) (width 0.2) (layer "B.Cu") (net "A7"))
 (segment (start 104.6 114.285) (end 105.645 114.285) (width 0.2) (layer "B.Cu") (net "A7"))
 (segment (start 105.645 115.555) (end 104.27 115.555) (width 0.2) (layer "F.Cu") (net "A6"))
 (via (at 105.645 115.555) (size 0.6) (drill 0.3) (layers "F.Cu" "B.Cu") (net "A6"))
 (segment (start 101.3 111.11) (end 104.1 111.11) (width 0.2) (layer "B.Cu") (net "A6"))
 (segment (start 104.1 115.555) (end 105.645 115.555) (width 0.2) (layer "B.Cu") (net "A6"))
 (segment (start 104.1 111.11) (end 104.1 115.555) (width 0.2) (layer "B.Cu") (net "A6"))
 (segment (start 105.645 116.825) (end 104.27 116.825) (width 0.2) (layer "F.Cu") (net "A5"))
 (via (at 105.645 116.825) (size 0.6) (drill 0.3) (layers "F.Cu" "B.Cu") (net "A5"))
 (segment (start 101.3 113.65) (end 103.6 113.65) (width 0.2) (layer "B.Cu") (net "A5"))
 (segment (start 103.6 113.65) (end 103.6 116.825) (width 0.2) (layer "B.Cu") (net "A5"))
 (segment (start 103.6 116.825) (end 105.645 116.825) (width 0.2) (layer "B.Cu") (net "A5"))
 (segment (start 105.645 118.095) (end 104.27 118.095) (width 0.2) (layer "F.Cu") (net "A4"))
 (via (at 105.645 118.095) (size 0.6) (drill 0.3) (layers "F.Cu" "B.Cu") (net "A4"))
 (segment (start 103.1 118.095) (end 105.645 118.095) (width 0.2) (layer "B.Cu") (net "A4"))
 (segment (start 101.3 116.19) (end 103.1 116.19) (width 0.2) (layer "B.Cu") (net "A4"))
 (segment (start 103.1 116.19) (end 103.1 118.095) (width 0.2) (layer "B.Cu") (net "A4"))
 (segment (start 105.645 119.365) (end 104.27 119.365) (width 0.2) (layer "F.Cu") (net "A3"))
 (via (at 105.645 119.365) (size 0.6) (drill 0.3) (layers "F.Cu" "B.Cu") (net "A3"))
 (segment (start 101.3 118.73) (end 102.6 118.73) (width 0.2) (layer "B.Cu") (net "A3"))
 (segment (start 102.6 119.365) (end 105.645 119.365) (width 0.2) (layer "B.Cu") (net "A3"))
 (segment (start 102.6 118.73) (end 102.6 119.365) (width 0.2) (layer "B.Cu") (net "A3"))
 (segment (start 105.645 120.635) (end 104.27 120.635) (width 0.2) (layer "F.Cu") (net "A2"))
 (via (at 105.645 120.635) (size 0.6) (drill 0.3) (layers "F.Cu" "B.Cu") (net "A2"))
 (segment (start 102.4 120.635) (end 105.645 120.635) (width 0.2) (layer "B.Cu") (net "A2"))
 (segment (start 101.3 121.27) (end 102.4 121.27) (width 0.2) (layer "B.Cu") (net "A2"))
 (segment (start 102.4 121.27) (end 102.4 120.635) (width 0.2) (layer "B.Cu") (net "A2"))
 (segment (start 105.645 121.905) (end 104.27 121.905) (width 0.2) (layer "F.Cu") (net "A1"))
 (via (at 105.645 121.905) (size 0.6) (drill 0.3) (layers "F.Cu" "B.Cu") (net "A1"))
 (segment (start 101.3 123.81) (end 102.85 123.81) (width 0.2) (layer "B.Cu") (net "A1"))
 (segment (start 102.85 123.81) (end 102.85 121.905) (width 0.2) (layer "B.Cu") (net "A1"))
 (segment (start 102.85 121.905) (end 105.645 121.905) (width 0.2) (layer "B.Cu") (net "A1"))
 (segment (start 105.645 123.175) (end 104.27 123.175) (width 0.2) (layer "F.Cu") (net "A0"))
 (via (at 105.645 123.175) (size 0.6) (drill 0.3) (layers "F.Cu" "B.Cu") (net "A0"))
 (segment (start 103.3 123.175) (end 105.645 123.175) (width 0.2) (layer "B.Cu") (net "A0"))
 (segment (start 103.3 126.35) (end 103.3 123.175) (width 0.2) (layer "B.Cu") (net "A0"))
 (segment (start 101.3 126.35) (end 103.3 126.35) (width 0.2) (layer "B.Cu") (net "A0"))
 (segment (start 105.645 124.445) (end 104.27 124.445) (width 0.2) (layer "F.Cu") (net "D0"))
 (via (at 105.645 124.445) (size 0.6) (drill 0.3) (layers "F.Cu" "B.Cu") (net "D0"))
 (segment (start 103.75 124.445) (end 105.645 124.445) (width 0.2) (layer "B.Cu") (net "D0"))
 (segment (start 103.75 128.889999) (end 103.75 124.445) (width 0.2) (layer "B.Cu") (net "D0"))
 (segment (start 101.3 128.889999) (end 103.75 128.889999) (width 0.2) (layer "B.Cu") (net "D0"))
 (segment (start 105.645 125.715) (end 104.27 125.715) (width 0.2) (layer "F.Cu") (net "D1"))
 (via (at 105.645 125.715) (size 0.6) (drill 0.3) (layers "F.Cu" "B.Cu") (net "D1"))
 (segment (start 101.3 131.43) (end 104.2 131.43) (width 0.2) (layer "B.Cu") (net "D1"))
 (segment (start 104.2 125.715) (end 105.645 125.715) (width 0.2) (layer "B.Cu") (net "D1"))
 (segment (start 104.2 131.43) (end 104.2 125.715) (width 0.2) (layer "B.Cu") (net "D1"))
 (segment (start 105.645 126.985) (end 104.27 126.985) (width 0.2) (layer "F.Cu") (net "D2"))
 (via (at 105.645 126.985) (size 0.6) (drill 0.3) (layers "F.Cu" "B.Cu") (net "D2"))
 (segment (start 104.65 126.985) (end 105.645 126.985) (width 0.2) (layer "B.Cu") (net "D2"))
 (segment (start 104.65 133.97) (end 104.65 126.985) (width 0.2) (layer "B.Cu") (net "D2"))
 (segment (start 101.3 133.97) (end 104.65 133.97) (width 0.2) (layer "B.Cu") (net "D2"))
 (segment (start 112.195 128.255) (end 113.57 128.255) (width 0.2) (layer "F.Cu") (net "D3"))
 (via (at 112.195 128.255) (size 0.6) (drill 0.3) (layers "F.Cu" "B.Cu") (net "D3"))
 (segment (start 112.74 128.255) (end 112.195 128.255) (width 0.2) (layer "B.Cu") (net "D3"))
 (segment (start 116.54 136.51) (end 112.74 136.51) (width 0.2) (layer "B.Cu") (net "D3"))
 (segment (start 112.74 136.51) (end 112.74 128.255) (width 0.2) (layer "B.Cu") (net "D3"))
 (segment (start 112.195 126.985) (end 113.57 126.985) (width 0.2) (layer "F.Cu") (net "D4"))
 (via (at 112.195 126.985) (size 0.6) (drill 0.3) (layers "F.Cu" "B.Cu") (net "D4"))
 (segment (start 116.54 133.97) (end 113.24 133.97) (width 0.2) (layer "B.Cu") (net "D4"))
 (segment (start 113.24 133.97) (end 113.24 126.985) (width 0.2) (layer "B.Cu") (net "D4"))
 (segment (start 113.24 126.985) (end 112.195 126.985) (width 0.2) (layer "B.Cu") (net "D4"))
 (segment (start 112.195 125.715) (end 113.57 125.715) (width 0.2) (layer "F.Cu") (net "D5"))
 (via (at 112.195 125.715) (size 0.6) (drill 0.3) (layers "F.Cu" "B.Cu") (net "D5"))
 (segment (start 113.74 125.715) (end 112.195 125.715) (width 0.2) (layer "B.Cu") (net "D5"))
 (segment (start 113.74 131.43) (end 113.74 125.715) (width 0.2) (layer "B.Cu") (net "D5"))
 (segment (start 116.54 131.43) (end 113.74 131.43) (width 0.2) (layer "B.Cu") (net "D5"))
 (segment (start 112.195 124.445) (end 113.57 124.445) (width 0.2) (layer "F.Cu") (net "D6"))
 (via (at 112.195 124.445) (size 0.6) (drill 0.3) (layers "F.Cu" "B.Cu") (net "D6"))
 (segment (start 116.54 128.889999) (end 114.24 128.889999) (width 0.2) (layer "B.Cu") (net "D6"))
 (segment (start 114.24 128.889999) (end 114.24 124.445) (width 0.2) (layer "B.Cu") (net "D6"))
 (segment (start 114.24 124.445) (end 112.195 124.445) (width 0.2) (layer "B.Cu") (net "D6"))
 (segment (start 112.195 123.175) (end 113.57 123.175) (width 0.2) (layer "F.Cu") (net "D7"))
 (via (at 112.195 123.175) (size 0.6) (drill 0.3) (layers "F.Cu" "B.Cu") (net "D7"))
 (segment (start 116.54 126.35) (end 114.74 126.35) (width 0.2) (layer "B.Cu") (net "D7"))
 (segment (start 114.74 126.35) (end 114.74 123.175) (width 0.2) (layer "B.Cu") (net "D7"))
 (segment (start 114.74 123.175) (end 112.195 123.175) (width 0.2) (layer "B.Cu") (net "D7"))
 (segment (start 112.195 120.635) (end 113.57 120.635) (width 0.2) (layer "F.Cu") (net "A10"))
 (via (at 112.195 120.635) (size 0.6) (drill 0.3) (layers "F.Cu" "B.Cu") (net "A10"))
 (segment (start 116.54 121.27) (end 115.24 121.27) (width 0.2) (layer "B.Cu") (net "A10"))
 (segment (start 115.24 120.635) (end 112.195 120.635) (width 0.2) (layer "B.Cu") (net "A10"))
 (segment (start 115.24 121.27) (end 115.24 120.635) (width 0.2) (layer "B.Cu") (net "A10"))
 (segment (start 112.195 119.365) (end 113.57 119.365) (width 0.2) (layer "F.Cu") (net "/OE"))
 (via (at 112.195 119.365) (size 0.6) (drill 0.3) (layers "F.Cu" "B.Cu") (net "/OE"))
 (segment (start 115.24 119.365) (end 112.195 119.365) (width 0.2) (layer "B.Cu") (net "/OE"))
 (segment (start 116.54 118.73) (end 115.24 118.73) (width 0.2) (layer "B.Cu") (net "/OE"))
 (segment (start 115.24 118.73) (end 115.24 119.365) (width 0.2) (layer "B.Cu") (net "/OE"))
 (segment (start 112.195 118.095) (end 113.57 118.095) (width 0.2) (layer "F.Cu") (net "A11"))
 (via (at 112.195 118.095) (size 0.6) (drill 0.3) (layers "F.Cu" "B.Cu") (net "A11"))
 (segment (start 114.74 116.19) (end 114.74 118.095) (width 0.2) (layer "B.Cu") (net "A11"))
 (segment (start 116.54 116.19) (end 114.74 116.19) (width 0.2) (layer "B.Cu") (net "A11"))
 (segment (start 114.74 118.095) (end 112.195 118.095) (width 0.2) (layer "B.Cu") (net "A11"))
 (segment (start 112.195 116.825) (end 113.57 116.825) (width 0.2) (layer "F.Cu") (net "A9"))
 (via (at 112.195 116.825) (size 0.6) (drill 0.3) (layers "F.Cu" "B.Cu") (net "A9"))
 (segment (start 114.24 113.65) (end 114.24 116.825) (width 0.2) (layer "B.Cu") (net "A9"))
 (segment (start 116.54 113.65) (end 114.24 113.65) (width 0.2) (layer "B.Cu") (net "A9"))
 (segment (start 114.24 116.825) (end 112.195 116.825) (width 0.2) (layer "B.Cu") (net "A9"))
 (segment (start 112.195 115.555) (end 113.57 115.555) (width 0.2) (layer "F.Cu") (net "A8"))
 (via (at 112.195 115.555) (size 0.6) (drill 0.3) (layers "F.Cu" "B.Cu") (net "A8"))
 (segment (start 116.54 111.11) (end 113.74 111.11) (width 0.2) (layer "B.Cu") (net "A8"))
 (segment (start 113.74 115.555) (end 112.195 115.555) (width 0.2) (layer "B.Cu") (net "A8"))
 (segment (start 113.74 111.11) (end 113.74 115.555) (width 0.2) (layer "B.Cu") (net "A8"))
 (segment (start 112.195 114.285) (end 113.57 114.285) (width 0.2) (layer "F.Cu") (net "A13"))
 (via (at 112.195 114.285) (size 0.6) (drill 0.3) (layers "F.Cu" "B.Cu") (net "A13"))
 (segment (start 113.24 108.57) (end 113.24 114.285) (width 0.2) (layer "B.Cu") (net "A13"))
 (segment (start 116.54 108.57) (end 113.24 108.57) (width 0.2) (layer "B.Cu") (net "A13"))
 (segment (start 113.24 114.285) (end 112.195 114.285) (width 0.2) (layer "B.Cu") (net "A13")))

